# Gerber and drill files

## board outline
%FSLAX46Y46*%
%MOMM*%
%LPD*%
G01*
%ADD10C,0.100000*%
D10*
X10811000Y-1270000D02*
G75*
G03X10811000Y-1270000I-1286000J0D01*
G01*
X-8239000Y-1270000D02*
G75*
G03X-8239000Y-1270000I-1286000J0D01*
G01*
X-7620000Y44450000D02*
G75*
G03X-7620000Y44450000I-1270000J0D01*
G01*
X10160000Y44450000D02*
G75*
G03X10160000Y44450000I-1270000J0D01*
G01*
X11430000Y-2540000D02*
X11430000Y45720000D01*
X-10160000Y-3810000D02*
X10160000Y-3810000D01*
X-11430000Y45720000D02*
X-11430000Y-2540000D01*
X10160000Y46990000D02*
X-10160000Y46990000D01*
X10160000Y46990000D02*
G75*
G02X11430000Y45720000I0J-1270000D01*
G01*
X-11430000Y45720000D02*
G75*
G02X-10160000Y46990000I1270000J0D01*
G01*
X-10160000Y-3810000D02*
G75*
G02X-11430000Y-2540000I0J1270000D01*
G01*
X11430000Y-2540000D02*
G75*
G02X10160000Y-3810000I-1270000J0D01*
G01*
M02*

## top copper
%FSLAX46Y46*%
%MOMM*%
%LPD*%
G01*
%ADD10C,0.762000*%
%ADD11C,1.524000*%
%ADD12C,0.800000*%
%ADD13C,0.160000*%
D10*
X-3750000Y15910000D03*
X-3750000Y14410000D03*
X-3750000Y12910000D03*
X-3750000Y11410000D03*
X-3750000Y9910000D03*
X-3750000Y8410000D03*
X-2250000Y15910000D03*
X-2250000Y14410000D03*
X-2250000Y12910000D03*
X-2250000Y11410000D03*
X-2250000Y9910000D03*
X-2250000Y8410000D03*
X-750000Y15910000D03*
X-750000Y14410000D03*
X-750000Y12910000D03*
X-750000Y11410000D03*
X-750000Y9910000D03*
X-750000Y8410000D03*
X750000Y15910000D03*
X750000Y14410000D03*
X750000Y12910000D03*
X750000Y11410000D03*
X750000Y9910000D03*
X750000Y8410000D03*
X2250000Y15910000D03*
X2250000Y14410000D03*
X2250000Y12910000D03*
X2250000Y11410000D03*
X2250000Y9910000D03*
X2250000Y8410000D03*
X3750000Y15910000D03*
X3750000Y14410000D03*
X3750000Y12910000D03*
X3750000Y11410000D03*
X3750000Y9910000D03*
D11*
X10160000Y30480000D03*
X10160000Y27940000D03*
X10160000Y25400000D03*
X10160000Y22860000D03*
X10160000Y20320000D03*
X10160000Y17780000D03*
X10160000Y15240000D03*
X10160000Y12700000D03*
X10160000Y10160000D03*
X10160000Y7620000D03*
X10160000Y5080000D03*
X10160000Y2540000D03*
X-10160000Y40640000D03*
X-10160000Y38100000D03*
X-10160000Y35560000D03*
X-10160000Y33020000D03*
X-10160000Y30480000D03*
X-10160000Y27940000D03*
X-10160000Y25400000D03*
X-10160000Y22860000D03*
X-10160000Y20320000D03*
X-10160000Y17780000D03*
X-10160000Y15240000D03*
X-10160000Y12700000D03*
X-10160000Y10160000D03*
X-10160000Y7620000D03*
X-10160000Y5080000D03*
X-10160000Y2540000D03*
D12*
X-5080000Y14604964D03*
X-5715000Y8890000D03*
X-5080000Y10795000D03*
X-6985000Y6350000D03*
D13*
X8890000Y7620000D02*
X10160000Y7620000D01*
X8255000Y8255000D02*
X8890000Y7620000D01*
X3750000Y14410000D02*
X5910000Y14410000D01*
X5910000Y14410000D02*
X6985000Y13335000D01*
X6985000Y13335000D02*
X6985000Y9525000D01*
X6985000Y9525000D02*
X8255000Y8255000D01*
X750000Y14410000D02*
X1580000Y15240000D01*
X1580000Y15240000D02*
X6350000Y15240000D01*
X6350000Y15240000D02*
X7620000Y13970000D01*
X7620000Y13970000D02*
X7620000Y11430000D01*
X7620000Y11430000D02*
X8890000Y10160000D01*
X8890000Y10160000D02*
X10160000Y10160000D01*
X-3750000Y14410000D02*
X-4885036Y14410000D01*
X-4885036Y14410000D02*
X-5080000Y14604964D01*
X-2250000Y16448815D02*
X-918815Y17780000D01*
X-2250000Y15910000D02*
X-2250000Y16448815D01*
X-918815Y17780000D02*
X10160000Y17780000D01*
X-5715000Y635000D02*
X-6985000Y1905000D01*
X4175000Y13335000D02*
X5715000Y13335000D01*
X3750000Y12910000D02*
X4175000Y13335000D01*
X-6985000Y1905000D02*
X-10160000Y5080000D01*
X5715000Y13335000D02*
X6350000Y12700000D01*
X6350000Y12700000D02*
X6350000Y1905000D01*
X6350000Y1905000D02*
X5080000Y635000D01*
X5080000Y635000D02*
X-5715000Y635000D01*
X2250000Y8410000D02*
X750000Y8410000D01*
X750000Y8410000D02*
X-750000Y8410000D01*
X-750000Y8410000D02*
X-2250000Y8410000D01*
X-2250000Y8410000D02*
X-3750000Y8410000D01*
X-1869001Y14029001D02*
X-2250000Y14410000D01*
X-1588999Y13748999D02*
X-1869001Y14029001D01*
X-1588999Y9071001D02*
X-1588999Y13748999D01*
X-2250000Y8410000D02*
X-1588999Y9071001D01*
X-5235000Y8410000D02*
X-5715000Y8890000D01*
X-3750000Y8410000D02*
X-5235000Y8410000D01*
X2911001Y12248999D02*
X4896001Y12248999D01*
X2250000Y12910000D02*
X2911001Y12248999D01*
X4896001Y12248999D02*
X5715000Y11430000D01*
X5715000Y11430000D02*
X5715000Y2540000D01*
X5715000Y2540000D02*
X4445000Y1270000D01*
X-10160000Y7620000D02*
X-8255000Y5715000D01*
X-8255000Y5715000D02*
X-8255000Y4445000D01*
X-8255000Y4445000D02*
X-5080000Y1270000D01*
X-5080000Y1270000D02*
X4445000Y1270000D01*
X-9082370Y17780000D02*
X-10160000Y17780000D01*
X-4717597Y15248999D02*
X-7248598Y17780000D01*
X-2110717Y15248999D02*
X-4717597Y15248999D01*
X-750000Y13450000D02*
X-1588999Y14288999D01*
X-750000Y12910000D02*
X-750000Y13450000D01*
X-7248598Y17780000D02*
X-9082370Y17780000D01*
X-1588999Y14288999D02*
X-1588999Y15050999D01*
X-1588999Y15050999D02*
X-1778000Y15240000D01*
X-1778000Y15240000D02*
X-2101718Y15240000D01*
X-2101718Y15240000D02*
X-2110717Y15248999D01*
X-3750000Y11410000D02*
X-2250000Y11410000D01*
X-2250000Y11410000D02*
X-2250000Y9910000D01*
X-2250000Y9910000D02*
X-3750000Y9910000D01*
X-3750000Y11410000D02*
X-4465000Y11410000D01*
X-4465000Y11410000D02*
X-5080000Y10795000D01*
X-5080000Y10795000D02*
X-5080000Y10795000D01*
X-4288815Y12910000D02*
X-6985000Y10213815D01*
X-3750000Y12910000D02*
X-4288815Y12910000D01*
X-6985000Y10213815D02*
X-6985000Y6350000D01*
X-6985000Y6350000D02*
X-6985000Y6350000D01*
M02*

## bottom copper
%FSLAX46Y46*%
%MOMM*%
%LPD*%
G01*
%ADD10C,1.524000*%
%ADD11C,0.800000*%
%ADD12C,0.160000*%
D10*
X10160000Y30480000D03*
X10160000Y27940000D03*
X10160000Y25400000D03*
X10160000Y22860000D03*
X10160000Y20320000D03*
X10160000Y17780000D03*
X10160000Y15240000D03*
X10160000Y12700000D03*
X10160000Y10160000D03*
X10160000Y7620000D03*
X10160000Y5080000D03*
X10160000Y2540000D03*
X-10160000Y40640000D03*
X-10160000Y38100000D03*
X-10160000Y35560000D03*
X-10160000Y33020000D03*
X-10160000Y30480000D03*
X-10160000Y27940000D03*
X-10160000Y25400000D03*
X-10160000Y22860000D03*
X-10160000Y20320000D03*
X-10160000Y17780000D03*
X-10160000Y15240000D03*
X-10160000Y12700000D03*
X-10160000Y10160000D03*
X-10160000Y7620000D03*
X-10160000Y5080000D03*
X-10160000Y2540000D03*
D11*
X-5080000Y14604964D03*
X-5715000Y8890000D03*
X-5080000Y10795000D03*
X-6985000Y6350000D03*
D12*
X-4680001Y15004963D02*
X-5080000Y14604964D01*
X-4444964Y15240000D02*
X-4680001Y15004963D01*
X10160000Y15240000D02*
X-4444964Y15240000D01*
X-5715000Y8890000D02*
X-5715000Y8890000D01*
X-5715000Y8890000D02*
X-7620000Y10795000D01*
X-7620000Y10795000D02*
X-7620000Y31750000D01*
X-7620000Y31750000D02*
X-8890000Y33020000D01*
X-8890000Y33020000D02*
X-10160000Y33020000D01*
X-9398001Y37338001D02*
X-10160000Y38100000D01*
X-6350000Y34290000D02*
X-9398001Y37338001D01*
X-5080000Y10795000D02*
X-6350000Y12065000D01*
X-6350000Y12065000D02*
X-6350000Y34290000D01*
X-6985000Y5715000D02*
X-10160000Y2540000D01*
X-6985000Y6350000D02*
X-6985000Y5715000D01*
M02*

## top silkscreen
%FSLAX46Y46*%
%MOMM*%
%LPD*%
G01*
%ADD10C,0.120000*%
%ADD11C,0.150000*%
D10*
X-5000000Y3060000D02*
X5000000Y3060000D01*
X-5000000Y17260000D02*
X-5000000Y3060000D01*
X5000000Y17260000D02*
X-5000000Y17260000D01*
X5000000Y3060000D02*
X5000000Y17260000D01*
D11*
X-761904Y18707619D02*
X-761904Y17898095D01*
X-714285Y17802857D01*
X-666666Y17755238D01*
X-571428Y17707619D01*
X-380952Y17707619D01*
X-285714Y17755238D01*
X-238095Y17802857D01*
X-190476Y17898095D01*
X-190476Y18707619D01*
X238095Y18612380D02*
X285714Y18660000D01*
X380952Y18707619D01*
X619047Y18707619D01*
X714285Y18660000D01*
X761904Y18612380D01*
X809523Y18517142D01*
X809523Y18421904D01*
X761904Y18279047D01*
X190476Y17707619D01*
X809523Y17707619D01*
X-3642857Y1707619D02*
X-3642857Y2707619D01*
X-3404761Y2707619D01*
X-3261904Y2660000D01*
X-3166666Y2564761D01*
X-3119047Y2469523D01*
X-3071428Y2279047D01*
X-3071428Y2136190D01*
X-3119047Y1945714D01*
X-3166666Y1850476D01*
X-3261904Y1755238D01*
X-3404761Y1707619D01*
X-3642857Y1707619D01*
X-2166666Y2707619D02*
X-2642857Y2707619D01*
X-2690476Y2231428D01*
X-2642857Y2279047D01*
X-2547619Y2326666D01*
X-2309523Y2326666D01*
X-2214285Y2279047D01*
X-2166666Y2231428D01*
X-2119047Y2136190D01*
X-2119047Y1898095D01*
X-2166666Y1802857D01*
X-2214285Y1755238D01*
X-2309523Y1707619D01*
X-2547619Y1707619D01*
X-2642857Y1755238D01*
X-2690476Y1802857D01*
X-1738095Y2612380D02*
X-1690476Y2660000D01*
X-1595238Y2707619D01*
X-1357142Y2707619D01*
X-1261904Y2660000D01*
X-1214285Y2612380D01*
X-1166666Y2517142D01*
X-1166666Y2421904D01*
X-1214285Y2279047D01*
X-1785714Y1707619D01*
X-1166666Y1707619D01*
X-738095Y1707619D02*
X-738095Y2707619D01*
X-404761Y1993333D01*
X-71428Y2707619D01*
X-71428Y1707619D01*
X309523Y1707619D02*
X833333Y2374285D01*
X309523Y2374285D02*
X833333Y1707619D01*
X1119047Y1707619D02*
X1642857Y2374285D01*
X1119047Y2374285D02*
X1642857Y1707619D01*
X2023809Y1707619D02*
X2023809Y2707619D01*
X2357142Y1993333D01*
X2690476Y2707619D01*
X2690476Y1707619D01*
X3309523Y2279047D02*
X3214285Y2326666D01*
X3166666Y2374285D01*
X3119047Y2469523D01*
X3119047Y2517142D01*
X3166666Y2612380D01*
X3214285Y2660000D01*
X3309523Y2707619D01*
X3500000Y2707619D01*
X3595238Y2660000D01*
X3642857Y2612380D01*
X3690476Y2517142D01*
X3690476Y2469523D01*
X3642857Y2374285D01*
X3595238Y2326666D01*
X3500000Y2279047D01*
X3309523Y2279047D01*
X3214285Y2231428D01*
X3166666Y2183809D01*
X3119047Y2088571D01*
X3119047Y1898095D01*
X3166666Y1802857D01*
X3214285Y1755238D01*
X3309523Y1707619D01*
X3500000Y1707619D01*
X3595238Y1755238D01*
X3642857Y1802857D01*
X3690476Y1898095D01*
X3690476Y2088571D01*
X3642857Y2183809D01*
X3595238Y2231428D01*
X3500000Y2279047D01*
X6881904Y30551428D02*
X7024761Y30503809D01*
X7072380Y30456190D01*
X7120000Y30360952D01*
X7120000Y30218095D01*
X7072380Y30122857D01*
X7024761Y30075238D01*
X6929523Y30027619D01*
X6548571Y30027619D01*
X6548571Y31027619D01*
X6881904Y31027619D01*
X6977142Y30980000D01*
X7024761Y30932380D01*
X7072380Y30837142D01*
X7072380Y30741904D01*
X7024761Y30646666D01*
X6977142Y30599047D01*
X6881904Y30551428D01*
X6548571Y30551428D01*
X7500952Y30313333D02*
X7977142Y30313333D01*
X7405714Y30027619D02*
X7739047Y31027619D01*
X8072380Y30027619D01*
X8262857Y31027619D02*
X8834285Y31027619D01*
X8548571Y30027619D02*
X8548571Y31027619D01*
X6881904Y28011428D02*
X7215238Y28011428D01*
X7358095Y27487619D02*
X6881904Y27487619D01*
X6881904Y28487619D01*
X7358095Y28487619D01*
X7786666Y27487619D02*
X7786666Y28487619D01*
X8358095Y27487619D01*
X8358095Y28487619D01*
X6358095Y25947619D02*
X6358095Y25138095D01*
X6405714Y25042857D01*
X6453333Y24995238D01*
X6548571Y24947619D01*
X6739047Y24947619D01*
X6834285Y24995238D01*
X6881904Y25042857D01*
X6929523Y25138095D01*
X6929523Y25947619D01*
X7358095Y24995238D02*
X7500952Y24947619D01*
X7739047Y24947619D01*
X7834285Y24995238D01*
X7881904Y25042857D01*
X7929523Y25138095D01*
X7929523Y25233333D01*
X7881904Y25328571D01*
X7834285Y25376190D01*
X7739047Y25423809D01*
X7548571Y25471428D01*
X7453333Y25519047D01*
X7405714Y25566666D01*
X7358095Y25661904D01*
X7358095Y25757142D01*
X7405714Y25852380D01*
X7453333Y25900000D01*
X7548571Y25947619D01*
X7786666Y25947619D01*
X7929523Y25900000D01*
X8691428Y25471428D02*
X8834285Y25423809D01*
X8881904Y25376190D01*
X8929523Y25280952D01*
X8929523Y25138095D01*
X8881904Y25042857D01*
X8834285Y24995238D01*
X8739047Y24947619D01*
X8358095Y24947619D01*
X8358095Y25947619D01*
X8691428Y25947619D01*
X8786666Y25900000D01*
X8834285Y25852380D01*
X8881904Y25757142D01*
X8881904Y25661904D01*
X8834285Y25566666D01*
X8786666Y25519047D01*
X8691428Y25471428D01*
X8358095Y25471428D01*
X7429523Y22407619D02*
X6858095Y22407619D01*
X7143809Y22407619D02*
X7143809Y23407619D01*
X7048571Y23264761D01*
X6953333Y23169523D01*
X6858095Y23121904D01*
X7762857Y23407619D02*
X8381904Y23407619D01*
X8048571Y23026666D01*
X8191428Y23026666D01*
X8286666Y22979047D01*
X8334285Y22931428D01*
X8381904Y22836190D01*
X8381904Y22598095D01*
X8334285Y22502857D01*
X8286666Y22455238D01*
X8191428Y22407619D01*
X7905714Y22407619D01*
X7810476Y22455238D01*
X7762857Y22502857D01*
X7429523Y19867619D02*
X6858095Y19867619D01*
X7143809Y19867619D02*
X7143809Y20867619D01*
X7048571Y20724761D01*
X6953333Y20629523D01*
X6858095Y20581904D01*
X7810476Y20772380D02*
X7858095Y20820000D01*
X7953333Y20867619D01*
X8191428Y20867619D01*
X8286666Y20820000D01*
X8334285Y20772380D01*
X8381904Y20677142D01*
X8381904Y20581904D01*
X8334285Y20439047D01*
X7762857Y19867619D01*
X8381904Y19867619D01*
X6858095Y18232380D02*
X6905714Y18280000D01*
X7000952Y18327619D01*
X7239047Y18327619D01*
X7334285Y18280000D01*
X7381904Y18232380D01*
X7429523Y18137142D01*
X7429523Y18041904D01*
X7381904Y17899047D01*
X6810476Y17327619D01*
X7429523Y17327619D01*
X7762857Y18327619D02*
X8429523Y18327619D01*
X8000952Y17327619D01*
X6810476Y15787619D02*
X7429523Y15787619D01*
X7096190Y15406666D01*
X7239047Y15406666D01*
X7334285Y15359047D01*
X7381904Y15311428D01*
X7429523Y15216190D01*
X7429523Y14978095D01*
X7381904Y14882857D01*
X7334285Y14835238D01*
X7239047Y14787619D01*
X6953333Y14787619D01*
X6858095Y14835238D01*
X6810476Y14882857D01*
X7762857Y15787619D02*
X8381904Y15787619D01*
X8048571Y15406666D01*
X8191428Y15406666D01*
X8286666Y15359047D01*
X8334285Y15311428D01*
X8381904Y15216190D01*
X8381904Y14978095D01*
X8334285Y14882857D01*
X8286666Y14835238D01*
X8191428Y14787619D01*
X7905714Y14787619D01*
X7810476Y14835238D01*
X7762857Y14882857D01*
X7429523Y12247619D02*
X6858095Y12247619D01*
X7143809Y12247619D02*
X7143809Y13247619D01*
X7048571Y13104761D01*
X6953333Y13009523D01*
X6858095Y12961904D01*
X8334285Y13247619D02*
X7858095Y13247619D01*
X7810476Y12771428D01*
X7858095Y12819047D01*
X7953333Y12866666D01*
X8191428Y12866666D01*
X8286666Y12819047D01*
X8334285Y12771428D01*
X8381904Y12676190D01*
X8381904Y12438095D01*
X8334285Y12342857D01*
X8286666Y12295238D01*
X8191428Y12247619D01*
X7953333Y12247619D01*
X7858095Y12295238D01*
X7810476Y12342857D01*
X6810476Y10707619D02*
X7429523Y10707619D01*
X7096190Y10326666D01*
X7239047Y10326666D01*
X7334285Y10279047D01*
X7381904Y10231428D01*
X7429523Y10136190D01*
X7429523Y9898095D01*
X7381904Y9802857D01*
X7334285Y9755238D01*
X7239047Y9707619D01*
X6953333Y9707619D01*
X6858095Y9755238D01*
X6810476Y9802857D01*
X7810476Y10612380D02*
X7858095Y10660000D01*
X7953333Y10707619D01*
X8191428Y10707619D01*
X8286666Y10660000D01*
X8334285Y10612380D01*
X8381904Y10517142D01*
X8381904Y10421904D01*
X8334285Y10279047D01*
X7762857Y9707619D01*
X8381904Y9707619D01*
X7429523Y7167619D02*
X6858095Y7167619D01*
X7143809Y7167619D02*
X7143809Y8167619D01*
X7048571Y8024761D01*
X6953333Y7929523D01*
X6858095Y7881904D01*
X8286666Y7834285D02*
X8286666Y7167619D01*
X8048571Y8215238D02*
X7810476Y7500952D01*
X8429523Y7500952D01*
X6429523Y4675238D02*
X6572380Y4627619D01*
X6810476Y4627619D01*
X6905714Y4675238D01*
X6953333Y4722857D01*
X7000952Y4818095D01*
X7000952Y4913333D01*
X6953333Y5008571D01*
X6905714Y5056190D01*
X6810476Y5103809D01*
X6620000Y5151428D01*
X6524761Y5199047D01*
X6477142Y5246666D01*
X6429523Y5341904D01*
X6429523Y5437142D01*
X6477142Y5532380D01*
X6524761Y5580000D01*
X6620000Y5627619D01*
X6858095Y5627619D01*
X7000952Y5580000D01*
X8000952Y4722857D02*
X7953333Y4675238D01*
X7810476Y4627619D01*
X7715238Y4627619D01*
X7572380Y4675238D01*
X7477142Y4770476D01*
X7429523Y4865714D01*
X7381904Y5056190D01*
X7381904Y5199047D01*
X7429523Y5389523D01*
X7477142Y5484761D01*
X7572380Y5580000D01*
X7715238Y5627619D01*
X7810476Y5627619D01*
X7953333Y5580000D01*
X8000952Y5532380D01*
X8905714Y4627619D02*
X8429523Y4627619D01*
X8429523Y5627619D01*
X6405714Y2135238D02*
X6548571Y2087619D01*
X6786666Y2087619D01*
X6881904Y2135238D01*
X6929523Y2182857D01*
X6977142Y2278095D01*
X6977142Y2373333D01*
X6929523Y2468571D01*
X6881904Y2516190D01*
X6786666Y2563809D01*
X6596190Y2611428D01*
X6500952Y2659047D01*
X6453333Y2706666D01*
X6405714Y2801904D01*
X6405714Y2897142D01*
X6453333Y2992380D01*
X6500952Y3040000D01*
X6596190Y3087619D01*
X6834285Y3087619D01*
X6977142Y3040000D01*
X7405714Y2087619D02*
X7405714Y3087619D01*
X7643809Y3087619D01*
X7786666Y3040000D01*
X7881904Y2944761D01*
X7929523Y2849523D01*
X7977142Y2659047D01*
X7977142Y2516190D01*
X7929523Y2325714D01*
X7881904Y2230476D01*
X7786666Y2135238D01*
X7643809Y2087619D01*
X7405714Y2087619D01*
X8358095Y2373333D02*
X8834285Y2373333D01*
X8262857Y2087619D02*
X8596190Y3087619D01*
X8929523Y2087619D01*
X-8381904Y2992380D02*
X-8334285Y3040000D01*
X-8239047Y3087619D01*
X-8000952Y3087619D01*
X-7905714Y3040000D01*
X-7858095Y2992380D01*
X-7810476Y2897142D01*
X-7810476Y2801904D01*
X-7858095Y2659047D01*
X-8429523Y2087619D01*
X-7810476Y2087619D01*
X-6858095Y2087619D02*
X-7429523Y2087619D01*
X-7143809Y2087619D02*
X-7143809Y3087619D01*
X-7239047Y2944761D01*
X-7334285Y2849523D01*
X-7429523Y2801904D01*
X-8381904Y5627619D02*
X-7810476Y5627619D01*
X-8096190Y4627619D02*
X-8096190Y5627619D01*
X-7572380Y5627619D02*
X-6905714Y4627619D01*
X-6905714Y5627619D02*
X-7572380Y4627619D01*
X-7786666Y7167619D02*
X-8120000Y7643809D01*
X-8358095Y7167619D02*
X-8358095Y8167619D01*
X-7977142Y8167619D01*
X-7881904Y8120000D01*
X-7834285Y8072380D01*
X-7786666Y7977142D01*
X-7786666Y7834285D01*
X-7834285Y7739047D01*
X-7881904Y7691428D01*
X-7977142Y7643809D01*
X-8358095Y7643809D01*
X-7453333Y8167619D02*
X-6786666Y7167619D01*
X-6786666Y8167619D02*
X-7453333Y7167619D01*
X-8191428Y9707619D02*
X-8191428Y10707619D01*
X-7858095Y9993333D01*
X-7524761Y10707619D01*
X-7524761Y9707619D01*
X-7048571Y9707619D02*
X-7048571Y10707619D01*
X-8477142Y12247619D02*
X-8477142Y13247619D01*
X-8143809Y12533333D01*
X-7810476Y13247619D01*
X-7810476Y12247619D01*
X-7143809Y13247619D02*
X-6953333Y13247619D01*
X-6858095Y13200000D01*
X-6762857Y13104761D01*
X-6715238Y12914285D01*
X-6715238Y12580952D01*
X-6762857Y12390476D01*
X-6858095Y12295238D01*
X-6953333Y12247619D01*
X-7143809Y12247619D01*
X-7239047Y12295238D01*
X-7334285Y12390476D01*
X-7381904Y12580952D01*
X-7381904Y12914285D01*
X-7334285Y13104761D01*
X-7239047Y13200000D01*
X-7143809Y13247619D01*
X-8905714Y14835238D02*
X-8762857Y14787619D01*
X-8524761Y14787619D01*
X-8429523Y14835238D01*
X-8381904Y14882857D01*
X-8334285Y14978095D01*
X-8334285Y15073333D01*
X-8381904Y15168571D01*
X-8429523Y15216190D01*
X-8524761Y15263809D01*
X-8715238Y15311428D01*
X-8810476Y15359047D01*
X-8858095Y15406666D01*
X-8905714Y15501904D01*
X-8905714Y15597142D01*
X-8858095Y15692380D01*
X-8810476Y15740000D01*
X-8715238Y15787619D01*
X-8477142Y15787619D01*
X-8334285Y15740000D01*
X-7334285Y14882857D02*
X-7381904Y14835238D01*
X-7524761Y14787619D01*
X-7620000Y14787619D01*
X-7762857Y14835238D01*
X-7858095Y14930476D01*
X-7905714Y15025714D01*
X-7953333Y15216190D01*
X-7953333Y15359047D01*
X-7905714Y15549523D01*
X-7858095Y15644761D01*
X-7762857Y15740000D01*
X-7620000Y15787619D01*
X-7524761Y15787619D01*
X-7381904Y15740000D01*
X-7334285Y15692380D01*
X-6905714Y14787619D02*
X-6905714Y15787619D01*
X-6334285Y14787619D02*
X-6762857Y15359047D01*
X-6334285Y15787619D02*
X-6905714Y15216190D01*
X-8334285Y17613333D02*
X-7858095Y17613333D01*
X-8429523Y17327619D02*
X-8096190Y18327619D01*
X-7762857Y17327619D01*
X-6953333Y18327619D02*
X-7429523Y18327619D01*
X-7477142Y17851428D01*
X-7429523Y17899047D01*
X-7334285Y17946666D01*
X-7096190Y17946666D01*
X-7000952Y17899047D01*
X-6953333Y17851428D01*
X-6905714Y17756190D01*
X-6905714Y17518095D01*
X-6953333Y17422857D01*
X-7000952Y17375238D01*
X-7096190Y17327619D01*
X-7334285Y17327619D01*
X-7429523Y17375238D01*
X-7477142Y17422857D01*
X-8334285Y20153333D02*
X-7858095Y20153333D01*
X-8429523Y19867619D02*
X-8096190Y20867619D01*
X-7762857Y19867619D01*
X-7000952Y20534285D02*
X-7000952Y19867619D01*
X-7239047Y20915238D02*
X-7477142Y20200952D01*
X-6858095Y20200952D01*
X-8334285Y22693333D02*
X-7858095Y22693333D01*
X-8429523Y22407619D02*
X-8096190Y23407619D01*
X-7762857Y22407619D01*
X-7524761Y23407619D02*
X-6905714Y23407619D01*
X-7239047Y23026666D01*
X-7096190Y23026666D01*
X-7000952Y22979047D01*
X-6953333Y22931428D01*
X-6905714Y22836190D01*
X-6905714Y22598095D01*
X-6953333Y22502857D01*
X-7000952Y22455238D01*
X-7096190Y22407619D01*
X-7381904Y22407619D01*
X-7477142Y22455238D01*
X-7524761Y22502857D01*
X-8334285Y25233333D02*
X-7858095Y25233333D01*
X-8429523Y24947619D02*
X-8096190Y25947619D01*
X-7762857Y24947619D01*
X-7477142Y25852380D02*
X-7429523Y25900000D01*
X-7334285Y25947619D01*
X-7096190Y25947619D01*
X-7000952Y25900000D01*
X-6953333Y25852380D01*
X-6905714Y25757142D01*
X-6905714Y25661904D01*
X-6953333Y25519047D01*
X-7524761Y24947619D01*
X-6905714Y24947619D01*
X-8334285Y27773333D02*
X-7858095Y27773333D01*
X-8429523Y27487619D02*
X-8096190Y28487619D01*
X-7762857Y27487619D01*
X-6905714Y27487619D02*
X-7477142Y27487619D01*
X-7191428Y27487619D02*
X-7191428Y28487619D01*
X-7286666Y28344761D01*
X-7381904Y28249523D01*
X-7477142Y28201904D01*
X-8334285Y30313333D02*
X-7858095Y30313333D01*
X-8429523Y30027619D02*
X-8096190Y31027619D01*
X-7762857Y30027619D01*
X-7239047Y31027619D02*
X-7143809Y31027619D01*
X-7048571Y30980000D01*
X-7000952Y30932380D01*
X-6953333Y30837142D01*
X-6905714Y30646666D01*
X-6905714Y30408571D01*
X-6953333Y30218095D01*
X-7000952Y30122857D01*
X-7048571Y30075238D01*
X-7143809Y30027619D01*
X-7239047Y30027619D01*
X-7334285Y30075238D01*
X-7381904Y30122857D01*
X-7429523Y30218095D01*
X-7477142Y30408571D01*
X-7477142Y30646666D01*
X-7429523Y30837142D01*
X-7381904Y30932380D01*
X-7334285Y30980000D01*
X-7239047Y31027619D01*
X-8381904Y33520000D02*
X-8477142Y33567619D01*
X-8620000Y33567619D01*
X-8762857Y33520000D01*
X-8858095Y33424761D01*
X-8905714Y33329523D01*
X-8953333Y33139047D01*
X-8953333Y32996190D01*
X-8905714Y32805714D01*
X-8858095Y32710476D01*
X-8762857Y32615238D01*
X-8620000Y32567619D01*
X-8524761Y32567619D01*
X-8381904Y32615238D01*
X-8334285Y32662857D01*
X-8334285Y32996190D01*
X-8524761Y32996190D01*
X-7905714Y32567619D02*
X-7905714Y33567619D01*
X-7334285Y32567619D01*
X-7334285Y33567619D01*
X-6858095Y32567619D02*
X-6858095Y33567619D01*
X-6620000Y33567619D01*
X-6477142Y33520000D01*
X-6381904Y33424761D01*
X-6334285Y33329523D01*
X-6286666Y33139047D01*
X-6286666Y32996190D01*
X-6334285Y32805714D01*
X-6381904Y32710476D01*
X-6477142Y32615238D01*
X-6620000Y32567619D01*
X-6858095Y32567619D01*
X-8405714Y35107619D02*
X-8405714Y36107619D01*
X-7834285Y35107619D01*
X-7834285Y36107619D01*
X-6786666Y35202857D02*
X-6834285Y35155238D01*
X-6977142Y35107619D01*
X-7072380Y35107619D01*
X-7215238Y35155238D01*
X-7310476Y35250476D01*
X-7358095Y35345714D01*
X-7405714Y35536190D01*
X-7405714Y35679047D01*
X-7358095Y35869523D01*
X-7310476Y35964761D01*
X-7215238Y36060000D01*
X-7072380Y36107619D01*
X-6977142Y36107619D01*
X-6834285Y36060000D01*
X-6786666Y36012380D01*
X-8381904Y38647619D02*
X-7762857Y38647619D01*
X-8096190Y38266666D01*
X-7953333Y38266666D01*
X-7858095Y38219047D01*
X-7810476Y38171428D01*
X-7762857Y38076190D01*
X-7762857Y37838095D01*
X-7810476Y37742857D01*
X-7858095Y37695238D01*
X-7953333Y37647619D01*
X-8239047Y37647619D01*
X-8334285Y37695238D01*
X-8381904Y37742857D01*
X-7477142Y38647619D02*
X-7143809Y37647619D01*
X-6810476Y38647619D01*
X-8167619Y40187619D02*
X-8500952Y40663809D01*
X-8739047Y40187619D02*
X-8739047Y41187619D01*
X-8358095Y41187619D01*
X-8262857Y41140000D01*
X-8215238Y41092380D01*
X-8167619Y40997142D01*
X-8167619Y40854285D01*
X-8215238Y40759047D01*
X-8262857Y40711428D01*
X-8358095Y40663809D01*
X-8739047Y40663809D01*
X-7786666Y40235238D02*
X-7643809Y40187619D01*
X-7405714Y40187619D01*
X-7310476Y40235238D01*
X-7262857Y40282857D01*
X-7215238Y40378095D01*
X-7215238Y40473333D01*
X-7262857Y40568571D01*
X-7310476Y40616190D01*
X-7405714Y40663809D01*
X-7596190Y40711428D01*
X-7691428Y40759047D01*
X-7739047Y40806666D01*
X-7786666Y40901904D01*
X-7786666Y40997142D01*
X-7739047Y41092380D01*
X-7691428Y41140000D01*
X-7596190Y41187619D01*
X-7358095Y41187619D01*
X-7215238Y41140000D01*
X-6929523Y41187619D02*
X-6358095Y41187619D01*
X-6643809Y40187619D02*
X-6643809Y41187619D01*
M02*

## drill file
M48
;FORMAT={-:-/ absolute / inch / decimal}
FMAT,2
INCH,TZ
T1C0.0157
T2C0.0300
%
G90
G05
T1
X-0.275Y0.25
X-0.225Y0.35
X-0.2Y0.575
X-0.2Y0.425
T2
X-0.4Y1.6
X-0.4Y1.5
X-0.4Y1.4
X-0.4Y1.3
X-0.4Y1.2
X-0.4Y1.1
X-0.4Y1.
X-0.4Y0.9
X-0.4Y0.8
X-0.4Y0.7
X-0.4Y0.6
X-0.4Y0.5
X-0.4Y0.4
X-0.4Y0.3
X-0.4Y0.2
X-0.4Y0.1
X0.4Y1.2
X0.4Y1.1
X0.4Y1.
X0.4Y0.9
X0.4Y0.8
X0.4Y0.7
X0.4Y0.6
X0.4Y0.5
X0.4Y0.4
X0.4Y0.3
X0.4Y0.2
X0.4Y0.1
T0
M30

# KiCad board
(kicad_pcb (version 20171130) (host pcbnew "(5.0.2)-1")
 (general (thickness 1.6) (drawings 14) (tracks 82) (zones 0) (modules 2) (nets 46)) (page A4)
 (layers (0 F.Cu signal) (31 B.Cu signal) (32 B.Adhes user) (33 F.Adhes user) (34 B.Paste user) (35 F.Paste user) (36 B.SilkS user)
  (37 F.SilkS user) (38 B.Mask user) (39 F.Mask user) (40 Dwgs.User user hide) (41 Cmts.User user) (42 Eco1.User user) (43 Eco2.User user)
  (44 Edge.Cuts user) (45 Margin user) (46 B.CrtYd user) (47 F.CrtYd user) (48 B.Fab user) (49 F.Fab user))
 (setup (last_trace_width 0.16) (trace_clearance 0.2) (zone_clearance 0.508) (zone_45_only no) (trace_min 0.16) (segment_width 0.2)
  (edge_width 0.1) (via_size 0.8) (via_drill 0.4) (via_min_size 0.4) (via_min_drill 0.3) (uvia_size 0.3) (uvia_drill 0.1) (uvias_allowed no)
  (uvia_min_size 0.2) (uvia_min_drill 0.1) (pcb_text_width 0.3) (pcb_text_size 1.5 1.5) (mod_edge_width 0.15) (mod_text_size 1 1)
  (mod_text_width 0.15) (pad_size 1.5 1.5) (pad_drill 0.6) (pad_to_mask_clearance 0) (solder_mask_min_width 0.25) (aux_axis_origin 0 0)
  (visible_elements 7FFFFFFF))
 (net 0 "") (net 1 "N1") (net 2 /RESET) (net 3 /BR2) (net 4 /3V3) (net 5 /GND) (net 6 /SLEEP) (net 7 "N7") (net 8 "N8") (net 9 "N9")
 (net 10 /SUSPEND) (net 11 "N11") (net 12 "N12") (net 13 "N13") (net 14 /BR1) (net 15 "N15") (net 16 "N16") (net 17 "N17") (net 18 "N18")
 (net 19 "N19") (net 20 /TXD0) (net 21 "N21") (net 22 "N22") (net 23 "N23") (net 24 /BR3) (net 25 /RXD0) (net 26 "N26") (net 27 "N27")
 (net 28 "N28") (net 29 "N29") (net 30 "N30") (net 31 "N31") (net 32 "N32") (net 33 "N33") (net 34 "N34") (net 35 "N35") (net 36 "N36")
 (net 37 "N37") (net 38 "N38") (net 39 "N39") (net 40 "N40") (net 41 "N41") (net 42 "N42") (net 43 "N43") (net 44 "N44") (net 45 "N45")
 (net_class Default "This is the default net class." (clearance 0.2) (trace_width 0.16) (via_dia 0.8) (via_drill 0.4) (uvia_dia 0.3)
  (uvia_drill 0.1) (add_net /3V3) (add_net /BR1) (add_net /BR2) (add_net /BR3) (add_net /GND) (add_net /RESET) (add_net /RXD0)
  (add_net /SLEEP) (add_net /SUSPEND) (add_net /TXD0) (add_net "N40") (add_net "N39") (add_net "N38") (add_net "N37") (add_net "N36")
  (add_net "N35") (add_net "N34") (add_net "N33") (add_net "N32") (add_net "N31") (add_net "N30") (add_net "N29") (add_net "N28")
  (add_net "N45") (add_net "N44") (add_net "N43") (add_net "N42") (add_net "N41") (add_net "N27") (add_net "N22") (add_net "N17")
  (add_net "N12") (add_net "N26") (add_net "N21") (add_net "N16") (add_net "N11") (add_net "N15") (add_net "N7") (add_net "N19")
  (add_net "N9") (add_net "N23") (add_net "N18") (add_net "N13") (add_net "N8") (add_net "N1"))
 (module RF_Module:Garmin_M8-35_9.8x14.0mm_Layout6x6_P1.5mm (layer F.Cu) (at 0 -10.16 180) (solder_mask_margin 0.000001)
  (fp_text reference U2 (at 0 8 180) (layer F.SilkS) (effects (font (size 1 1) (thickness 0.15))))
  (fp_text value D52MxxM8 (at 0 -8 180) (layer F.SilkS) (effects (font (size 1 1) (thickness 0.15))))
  (fp_line (start 5 -7.1) (end -5 -7.1) (layer F.SilkS) (width 0.12))
  (fp_line (start 5 7.1) (end 5 -7.1) (layer F.SilkS) (width 0.12))
  (fp_line (start -5 7.1) (end 5 7.1) (layer F.SilkS) (width 0.12))
  (fp_line (start -5 -7.1) (end -5 7.1) (layer F.SilkS) (width 0.12))
  (pad F6 smd circle (at 3.75 5.75 180) (size 0.762 0.762) (layers F.Cu F.Mask) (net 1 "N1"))
  (pad E6 smd circle (at 3.75 4.25 180) (size 0.762 0.762) (layers F.Cu F.Mask) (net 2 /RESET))
  (pad D6 smd circle (at 3.75 2.75 180) (size 0.762 0.762) (layers F.Cu F.Mask) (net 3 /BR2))
  (pad C6 smd circle (at 3.75 1.25 180) (size 0.762 0.762) (layers F.Cu F.Mask) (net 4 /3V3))
  (pad B6 smd circle (at 3.75 -0.25 180) (size 0.762 0.762) (layers F.Cu F.Mask) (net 4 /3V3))
  (pad A6 smd circle (at 3.75 -1.75 180) (size 0.762 0.762) (layers F.Cu F.Mask) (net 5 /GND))
  (pad F5 smd circle (at 2.25 5.75 180) (size 0.762 0.762) (layers F.Cu F.Mask) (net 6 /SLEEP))
  (pad E5 smd circle (at 2.25 4.25 180) (size 0.762 0.762) (layers F.Cu F.Mask) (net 5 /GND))
  (pad D5 smd circle (at 2.25 2.75 180) (size 0.762 0.762) (layers F.Cu F.Mask) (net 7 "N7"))
  (pad C5 smd circle (at 2.25 1.25 180) (size 0.762 0.762) (layers F.Cu F.Mask) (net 4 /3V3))
  (pad B5 smd circle (at 2.25 -0.25 180) (size 0.762 0.762) (layers F.Cu F.Mask) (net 4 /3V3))
  (pad A5 smd circle (at 2.25 -1.75 180) (size 0.762 0.762) (layers F.Cu F.Mask) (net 5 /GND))
  (pad F4 smd circle (at 0.75 5.75 180) (size 0.762 0.762) (layers F.Cu F.Mask) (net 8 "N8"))
  (pad E4 smd circle (at 0.75 4.25 180) (size 0.762 0.762) (layers F.Cu F.Mask) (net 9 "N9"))
  (pad D4 smd circle (at 0.75 2.75 180) (size 0.762 0.762) (layers F.Cu F.Mask) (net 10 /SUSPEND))
  (pad C4 smd circle (at 0.75 1.25 180) (size 0.762 0.762) (layers F.Cu F.Mask) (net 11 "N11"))
  (pad B4 smd circle (at 0.75 -0.25 180) (size 0.762 0.762) (layers F.Cu F.Mask) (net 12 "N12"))
  (pad A4 smd circle (at 0.75 -1.75 180) (size 0.762 0.762) (layers F.Cu F.Mask) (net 5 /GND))
  (pad F3 smd circle (at -0.75 5.75 180) (size 0.762 0.762) (layers F.Cu F.Mask) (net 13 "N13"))
  (pad E3 smd circle (at -0.75 4.25 180) (size 0.762 0.762) (layers F.Cu F.Mask) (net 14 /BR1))
  (pad D3 smd circle (at -0.75 2.75 180) (size 0.762 0.762) (layers F.Cu F.Mask) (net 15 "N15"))
  (pad C3 smd circle (at -0.75 1.25 180) (size 0.762 0.762) (layers F.Cu F.Mask) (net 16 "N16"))
  (pad B3 smd circle (at -0.75 -0.25 180) (size 0.762 0.762) (layers F.Cu F.Mask) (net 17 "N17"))
  (pad A3 smd circle (at -0.75 -1.75 180) (size 0.762 0.762) (layers F.Cu F.Mask) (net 5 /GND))
  (pad F2 smd circle (at -2.25 5.75 180) (size 0.762 0.762) (layers F.Cu F.Mask) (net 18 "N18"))
  (pad E2 smd circle (at -2.25 4.25 180) (size 0.762 0.762) (layers F.Cu F.Mask) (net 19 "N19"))
  (pad D2 smd circle (at -2.25 2.75 180) (size 0.762 0.762) (layers F.Cu F.Mask) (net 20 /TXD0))
  (pad C2 smd circle (at -2.25 1.25 180) (size 0.762 0.762) (layers F.Cu F.Mask) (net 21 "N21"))
  (pad B2 smd circle (at -2.25 -0.25 180) (size 0.762 0.762) (layers F.Cu F.Mask) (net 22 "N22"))
  (pad A2 smd circle (at -2.25 -1.75 180) (size 0.762 0.762) (layers F.Cu F.Mask) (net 5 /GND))
  (pad F1 smd circle (at -3.75 5.75 180) (size 0.762 0.762) (layers F.Cu F.Mask) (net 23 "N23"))
  (pad E1 smd circle (at -3.75 4.25 180) (size 0.762 0.762) (layers F.Cu F.Mask) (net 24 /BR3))
  (pad D1 smd circle (at -3.75 2.75 180) (size 0.762 0.762) (layers F.Cu F.Mask) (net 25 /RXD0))
  (pad C1 smd circle (at -3.75 1.25 180) (size 0.762 0.762) (layers F.Cu F.Mask) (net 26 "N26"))
  (pad B1 smd circle (at -3.75 -0.25 180) (size 0.762 0.762) (layers F.Cu F.Mask) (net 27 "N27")))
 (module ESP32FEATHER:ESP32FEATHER (layer F.Cu) (at 0 0)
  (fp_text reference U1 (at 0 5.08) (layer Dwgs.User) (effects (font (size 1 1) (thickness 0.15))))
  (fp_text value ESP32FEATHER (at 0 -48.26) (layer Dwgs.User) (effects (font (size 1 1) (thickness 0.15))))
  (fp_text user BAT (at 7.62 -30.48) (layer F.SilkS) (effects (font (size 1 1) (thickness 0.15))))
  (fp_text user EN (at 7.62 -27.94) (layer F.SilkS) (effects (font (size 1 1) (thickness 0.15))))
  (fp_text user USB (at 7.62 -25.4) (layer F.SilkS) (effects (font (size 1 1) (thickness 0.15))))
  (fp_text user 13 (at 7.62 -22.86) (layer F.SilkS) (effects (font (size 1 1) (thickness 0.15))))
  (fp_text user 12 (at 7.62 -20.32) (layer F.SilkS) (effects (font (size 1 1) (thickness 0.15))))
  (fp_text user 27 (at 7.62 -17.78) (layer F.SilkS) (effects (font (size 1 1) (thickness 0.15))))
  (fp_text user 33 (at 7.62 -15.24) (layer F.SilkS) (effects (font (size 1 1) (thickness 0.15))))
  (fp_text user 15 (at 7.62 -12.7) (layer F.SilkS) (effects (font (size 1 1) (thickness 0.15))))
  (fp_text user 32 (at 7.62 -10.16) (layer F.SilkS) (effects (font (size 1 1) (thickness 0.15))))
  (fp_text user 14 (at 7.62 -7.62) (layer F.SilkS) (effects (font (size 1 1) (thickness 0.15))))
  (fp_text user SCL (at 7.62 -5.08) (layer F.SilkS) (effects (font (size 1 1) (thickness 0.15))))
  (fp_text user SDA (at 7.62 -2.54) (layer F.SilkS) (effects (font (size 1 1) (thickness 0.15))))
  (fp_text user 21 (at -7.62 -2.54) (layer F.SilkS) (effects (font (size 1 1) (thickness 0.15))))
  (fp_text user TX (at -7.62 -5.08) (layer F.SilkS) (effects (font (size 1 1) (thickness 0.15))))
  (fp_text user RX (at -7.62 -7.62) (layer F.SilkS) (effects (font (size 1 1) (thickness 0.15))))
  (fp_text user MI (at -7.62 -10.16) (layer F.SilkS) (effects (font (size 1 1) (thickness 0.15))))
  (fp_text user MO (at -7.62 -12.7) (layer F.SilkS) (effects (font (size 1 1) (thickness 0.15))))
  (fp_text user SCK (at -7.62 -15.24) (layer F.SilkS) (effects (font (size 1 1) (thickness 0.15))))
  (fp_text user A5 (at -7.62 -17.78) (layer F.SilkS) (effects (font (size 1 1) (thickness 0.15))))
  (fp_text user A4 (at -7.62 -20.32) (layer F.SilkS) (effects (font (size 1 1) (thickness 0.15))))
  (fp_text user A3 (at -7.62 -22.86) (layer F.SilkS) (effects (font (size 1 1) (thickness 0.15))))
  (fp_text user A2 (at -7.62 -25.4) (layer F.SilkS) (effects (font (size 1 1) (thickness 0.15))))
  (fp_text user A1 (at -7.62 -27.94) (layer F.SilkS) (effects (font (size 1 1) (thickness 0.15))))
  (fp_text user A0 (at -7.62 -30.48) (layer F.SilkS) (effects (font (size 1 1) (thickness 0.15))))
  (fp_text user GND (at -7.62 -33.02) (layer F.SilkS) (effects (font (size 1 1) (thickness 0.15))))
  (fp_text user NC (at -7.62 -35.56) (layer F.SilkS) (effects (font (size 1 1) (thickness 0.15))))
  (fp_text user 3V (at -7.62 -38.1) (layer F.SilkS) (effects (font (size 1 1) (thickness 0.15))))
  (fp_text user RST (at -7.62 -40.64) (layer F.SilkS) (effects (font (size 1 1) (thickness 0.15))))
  (pad 28 thru_hole circle (at 10.16 -30.48) (size 1.524 1.524) (drill 0.762) (layers *.Cu *.Mask) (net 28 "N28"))
  (pad 27 thru_hole circle (at 10.16 -27.94) (size 1.524 1.524) (drill 0.762) (layers *.Cu *.Mask) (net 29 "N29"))
  (pad 26 thru_hole circle (at 10.16 -25.4) (size 1.524 1.524) (drill 0.762) (layers *.Cu *.Mask) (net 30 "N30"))
  (pad 25 thru_hole circle (at 10.16 -22.86) (size 1.524 1.524) (drill 0.762) (layers *.Cu *.Mask) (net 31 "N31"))
  (pad 24 thru_hole circle (at 10.16 -20.32) (size 1.524 1.524) (drill 0.762) (layers *.Cu *.Mask) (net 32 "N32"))
  (pad 23 thru_hole circle (at 10.16 -17.78) (size 1.524 1.524) (drill 0.762) (layers *.Cu *.Mask) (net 6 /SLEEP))
  (pad 22 thru_hole circle (at 10.16 -15.24) (size 1.524 1.524) (drill 0.762) (layers *.Cu *.Mask) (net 2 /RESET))
  (pad 21 thru_hole circle (at 10.16 -12.7) (size 1.524 1.524) (drill 0.762) (layers *.Cu *.Mask) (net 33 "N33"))
  (pad 20 thru_hole circle (at 10.16 -10.16) (size 1.524 1.524) (drill 0.762) (layers *.Cu *.Mask) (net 14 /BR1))
  (pad 19 thru_hole circle (at 10.16 -7.62) (size 1.524 1.524) (drill 0.762) (layers *.Cu *.Mask) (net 24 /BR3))
  (pad 18 thru_hole circle (at 10.16 -5.08) (size 1.524 1.524) (drill 0.762) (layers *.Cu *.Mask) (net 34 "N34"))
  (pad 17 thru_hole circle (at 10.16 -2.54) (size 1.524 1.524) (drill 0.762) (layers *.Cu *.Mask) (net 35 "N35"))
  (pad 16 thru_hole circle (at -10.16 -40.64) (size 1.524 1.524) (drill 0.762) (layers *.Cu *.Mask) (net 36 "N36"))
  (pad 15 thru_hole circle (at -10.16 -38.1) (size 1.524 1.524) (drill 0.762) (layers *.Cu *.Mask) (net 4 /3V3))
  (pad 14 thru_hole circle (at -10.16 -35.56) (size 1.524 1.524) (drill 0.762) (layers *.Cu *.Mask) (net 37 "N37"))
  (pad 13 thru_hole circle (at -10.16 -33.02) (size 1.524 1.524) (drill 0.762) (layers *.Cu *.Mask) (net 5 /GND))
  (pad 12 thru_hole circle (at -10.16 -30.48) (size 1.524 1.524) (drill 0.762) (layers *.Cu *.Mask) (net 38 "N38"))
  (pad 11 thru_hole circle (at -10.16 -27.94) (size 1.524 1.524) (drill 0.762) (layers *.Cu *.Mask) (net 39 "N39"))
  (pad 10 thru_hole circle (at -10.16 -25.4) (size 1.524 1.524) (drill 0.762) (layers *.Cu *.Mask) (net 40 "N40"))
  (pad 9 thru_hole circle (at -10.16 -22.86) (size 1.524 1.524) (drill 0.762) (layers *.Cu *.Mask) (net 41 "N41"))
  (pad 8 thru_hole circle (at -10.16 -20.32) (size 1.524 1.524) (drill 0.762) (layers *.Cu *.Mask) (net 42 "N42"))
  (pad 7 thru_hole circle (at -10.16 -17.78) (size 1.524 1.524) (drill 0.762) (layers *.Cu *.Mask) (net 10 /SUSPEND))
  (pad 6 thru_hole circle (at -10.16 -15.24) (size 1.524 1.524) (drill 0.762) (layers *.Cu *.Mask) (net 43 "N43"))
  (pad 5 thru_hole circle (at -10.16 -12.7) (size 1.524 1.524) (drill 0.762) (layers *.Cu *.Mask) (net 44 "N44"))
  (pad 4 thru_hole circle (at -10.16 -10.16) (size 1.524 1.524) (drill 0.762) (layers *.Cu *.Mask) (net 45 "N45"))
  (pad 3 thru_hole circle (at -10.16 -7.62) (size 1.524 1.524) (drill 0.762) (layers *.Cu *.Mask) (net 20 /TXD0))
  (pad 2 thru_hole circle (at -10.16 -5.08) (size 1.524 1.524) (drill 0.762) (layers *.Cu *.Mask) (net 25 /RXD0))
  (pad 1 thru_hole circle (at -10.16 -2.54) (size 1.524 1.524) (drill 0.762) (layers *.Cu *.Mask) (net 3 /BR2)))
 (gr_circle (center 9.525 1.27) (end 10.811 1.27) (layer Edge.Cuts) (width 0.1))
 (gr_circle (center -9.525 1.27) (end -8.239 1.27) (layer Edge.Cuts) (width 0.1))
 (gr_circle (center -8.89 -44.45) (end -8.89 -43.18) (layer Edge.Cuts) (width 0.1))
 (gr_circle (center 8.89 -44.45) (end 8.89 -43.18) (layer Edge.Cuts) (width 0.1))
 (gr_line (start 11.43 2.54) (end 11.43 -45.72) (layer Edge.Cuts) (width 0.1))
 (gr_line (start -10.16 3.81) (end 10.16 3.81) (layer Edge.Cuts) (width 0.1))
 (gr_line (start -11.43 -45.72) (end -11.43 2.54) (layer Edge.Cuts) (width 0.1))
 (gr_line (start 10.16 -46.99) (end -10.16 -46.99) (layer Edge.Cuts) (width 0.1))
 (gr_arc (start 10.16 -45.72) (end 11.43 -45.72) (angle -90) (layer Edge.Cuts) (width 0.1))
 (gr_arc (start -10.16 -45.72) (end -10.16 -46.99) (angle -90) (layer Edge.Cuts) (width 0.1))
 (gr_arc (start -10.16 2.54) (end -11.43 2.54) (angle -90) (layer Edge.Cuts) (width 0.1))
 (gr_arc (start 10.16 2.54) (end 10.16 3.81) (angle -90) (layer Edge.Cuts) (width 0.1))
 (segment (start 8.89 -7.62) (end 10.16 -7.62) (width 0.16) (layer F.Cu) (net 24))
 (segment (start 8.255 -8.255) (end 8.89 -7.62) (width 0.16) (layer F.Cu) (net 24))
 (segment (start 3.75 -14.41) (end 5.91 -14.41) (width 0.16) (layer F.Cu) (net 24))
 (segment (start 5.91 -14.41) (end 6.985 -13.335) (width 0.16) (layer F.Cu) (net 24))
 (segment (start 6.985 -13.335) (end 6.985 -9.525) (width 0.16) (layer F.Cu) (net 24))
 (segment (start 6.985 -9.525) (end 8.255 -8.255) (width 0.16) (layer F.Cu) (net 24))
 (segment (start 0.75 -14.41) (end 1.58 -15.24) (width 0.16) (layer F.Cu) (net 14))
 (segment (start 1.58 -15.24) (end 6.35 -15.24) (width 0.16) (layer F.Cu) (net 14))
 (segment (start 6.35 -15.24) (end 7.62 -13.97) (width 0.16) (layer F.Cu) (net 14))
 (segment (start 7.62 -13.97) (end 7.62 -11.43) (width 0.16) (layer F.Cu) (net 14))
 (segment (start 7.62 -11.43) (end 8.89 -10.16) (width 0.16) (layer F.Cu) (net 14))
 (segment (start 8.89 -10.16) (end 10.16 -10.16) (width 0.16) (layer F.Cu) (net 14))
 (segment (start -4.680001 -15.004963) (end -5.08 -14.604964) (width 0.16) (layer B.Cu) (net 2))
 (segment (start -4.444964 -15.24) (end -4.680001 -15.004963) (width 0.16) (layer B.Cu) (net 2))
 (segment (start -3.75 -14.41) (end -4.885036 -14.41) (width 0.16) (layer F.Cu) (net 2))
 (via (at -5.08 -14.604964) (size 0.8) (drill 0.4) (layers F.Cu B.Cu) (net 2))
 (segment (start -4.885036 -14.41) (end -5.08 -14.604964) (width 0.16) (layer F.Cu) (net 2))
 (segment (start 10.16 -15.24) (end -4.444964 -15.24) (width 0.16) (layer B.Cu) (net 2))
 (segment (start -2.25 -16.448815) (end -0.918815 -17.78) (width 0.16) (layer F.Cu) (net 6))
 (segment (start -2.25 -15.91) (end -2.25 -16.448815) (width 0.16) (layer F.Cu) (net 6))
 (segment (start -0.918815 -17.78) (end 10.16 -17.78) (width 0.16) (layer F.Cu) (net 6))
 (segment (start -5.715 -0.635) (end -6.985 -1.905) (width 0.16) (layer F.Cu) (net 25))
 (segment (start 4.175 -13.335) (end 5.715 -13.335) (width 0.16) (layer F.Cu) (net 25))
 (segment (start 3.75 -12.91) (end 4.175 -13.335) (width 0.16) (layer F.Cu) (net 25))
 (segment (start -6.985 -1.905) (end -10.16 -5.08) (width 0.16) (layer F.Cu) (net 25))
 (segment (start 5.715 -13.335) (end 6.35 -12.7) (width 0.16) (layer F.Cu) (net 25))
 (segment (start 6.35 -12.7) (end 6.35 -1.905) (width 0.16) (layer F.Cu) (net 25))
 (segment (start 6.35 -1.905) (end 5.08 -0.635) (width 0.16) (layer F.Cu) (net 25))
 (segment (start 5.08 -0.635) (end -5.715 -0.635) (width 0.16) (layer F.Cu) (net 25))
 (segment (start 2.25 -8.41) (end 0.75 -8.41) (width 0.16) (layer F.Cu) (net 5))
 (segment (start 0.75 -8.41) (end -0.75 -8.41) (width 0.16) (layer F.Cu) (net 5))
 (segment (start -0.75 -8.41) (end -2.25 -8.41) (width 0.16) (layer F.Cu) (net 5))
 (segment (start -2.25 -8.41) (end -3.75 -8.41) (width 0.16) (layer F.Cu) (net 5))
 (segment (start -1.869001 -14.029001) (end -2.25 -14.41) (width 0.16) (layer F.Cu) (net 5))
 (segment (start -1.588999 -13.748999) (end -1.869001 -14.029001) (width 0.16) (layer F.Cu) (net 5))
 (segment (start -1.588999 -9.071001) (end -1.588999 -13.748999) (width 0.16) (layer F.Cu) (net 5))
 (segment (start -2.25 -8.41) (end -1.588999 -9.071001) (width 0.16) (layer F.Cu) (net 5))
 (segment (start -5.715 -8.89) (end -5.715 -8.89) (width 0.16) (layer B.Cu) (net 5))
 (via (at -5.715 -8.89) (size 0.8) (drill 0.4) (layers F.Cu B.Cu) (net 5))
 (segment (start -5.715 -8.89) (end -7.62 -10.795) (width 0.16) (layer B.Cu) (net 5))
 (segment (start -7.62 -10.795) (end -7.62 -31.75) (width 0.16) (layer B.Cu) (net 5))
 (segment (start -7.62 -31.75) (end -8.89 -33.02) (width 0.16) (layer B.Cu) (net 5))
 (segment (start -8.89 -33.02) (end -10.16 -33.02) (width 0.16) (layer B.Cu) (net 5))
 (segment (start -5.235 -8.41) (end -5.715 -8.89) (width 0.16) (layer F.Cu) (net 5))
 (segment (start -3.75 -8.41) (end -5.235 -8.41) (width 0.16) (layer F.Cu) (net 5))
 (segment (start 2.911001 -12.248999) (end 4.896001 -12.248999) (width 0.16) (layer F.Cu) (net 20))
 (segment (start 2.25 -12.91) (end 2.911001 -12.248999) (width 0.16) (layer F.Cu) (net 20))
 (segment (start 4.896001 -12.248999) (end 5.715 -11.43) (width 0.16) (layer F.Cu) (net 20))
 (segment (start 5.715 -11.43) (end 5.715 -2.54) (width 0.16) (layer F.Cu) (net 20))
 (segment (start 5.715 -2.54) (end 4.445 -1.27) (width 0.16) (layer F.Cu) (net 20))
 (segment (start -10.16 -7.62) (end -8.255 -5.715) (width 0.16) (layer F.Cu) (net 20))
 (segment (start -8.255 -5.715) (end -8.255 -4.445) (width 0.16) (layer F.Cu) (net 20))
 (segment (start -8.255 -4.445) (end -5.08 -1.27) (width 0.16) (layer F.Cu) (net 20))
 (segment (start -5.08 -1.27) (end 4.445 -1.27) (width 0.16) (layer F.Cu) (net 20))
 (segment (start -9.08237 -17.78) (end -10.16 -17.78) (width 0.16) (layer F.Cu) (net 10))
 (segment (start -4.717597 -15.248999) (end -7.248598 -17.78) (width 0.16) (layer F.Cu) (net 10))
 (segment (start -2.110717 -15.248999) (end -4.717597 -15.248999) (width 0.16) (layer F.Cu) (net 10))
 (segment (start -0.75 -13.45) (end -1.588999 -14.288999) (width 0.16) (layer F.Cu) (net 10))
 (segment (start -0.75 -12.91) (end -0.75 -13.45) (width 0.16) (layer F.Cu) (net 10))
 (segment (start -7.248598 -17.78) (end -9.08237 -17.78) (width 0.16) (layer F.Cu) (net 10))
 (segment (start -1.588999 -14.288999) (end -1.588999 -15.050999) (width 0.16) (layer F.Cu) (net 10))
 (segment (start -1.588999 -15.050999) (end -1.778 -15.24) (width 0.16) (layer F.Cu) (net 10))
 (segment (start -1.778 -15.24) (end -2.101718 -15.24) (width 0.16) (layer F.Cu) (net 10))
 (segment (start -2.101718 -15.24) (end -2.110717 -15.248999) (width 0.16) (layer F.Cu) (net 10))
 (segment (start -3.75 -11.41) (end -2.25 -11.41) (width 0.16) (layer F.Cu) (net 4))
 (segment (start -2.25 -11.41) (end -2.25 -9.91) (width 0.16) (layer F.Cu) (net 4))
 (segment (start -2.25 -9.91) (end -3.75 -9.91) (width 0.16) (layer F.Cu) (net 4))
 (segment (start -3.75 -11.41) (end -4.465 -11.41) (width 0.16) (layer F.Cu) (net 4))
 (segment (start -4.465 -11.41) (end -5.08 -10.795) (width 0.16) (layer F.Cu) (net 4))
 (segment (start -5.08 -10.795) (end -5.08 -10.795) (width 0.16) (layer F.Cu) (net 4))
 (via (at -5.08 -10.795) (size 0.8) (drill 0.4) (layers F.Cu B.Cu) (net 4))
 (segment (start -9.398001 -37.338001) (end -10.16 -38.1) (width 0.16) (layer B.Cu) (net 4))
 (segment (start -6.35 -34.29) (end -9.398001 -37.338001) (width 0.16) (layer B.Cu) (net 4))
 (segment (start -5.08 -10.795) (end -6.35 -12.065) (width 0.16) (layer B.Cu) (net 4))
 (segment (start -6.35 -12.065) (end -6.35 -34.29) (width 0.16) (layer B.Cu) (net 4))
 (segment (start -4.288815 -12.91) (end -6.985 -10.213815) (width 0.16) (layer F.Cu) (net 3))
 (segment (start -3.75 -12.91) (end -4.288815 -12.91) (width 0.16) (layer F.Cu) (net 3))
 (segment (start -6.985 -10.213815) (end -6.985 -6.35) (width 0.16) (layer F.Cu) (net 3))
 (segment (start -6.985 -6.35) (end -6.985 -6.35) (width 0.16) (layer F.Cu) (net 3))
 (via (at -6.985 -6.35) (size 0.8) (drill 0.4) (layers F.Cu B.Cu) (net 3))
 (segment (start -6.985 -5.715) (end -10.16 -2.54) (width 0.16) (layer B.Cu) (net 3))
 (segment (start -6.985 -6.35) (end -6.985 -5.715) (width 0.16) (layer B.Cu) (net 3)))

